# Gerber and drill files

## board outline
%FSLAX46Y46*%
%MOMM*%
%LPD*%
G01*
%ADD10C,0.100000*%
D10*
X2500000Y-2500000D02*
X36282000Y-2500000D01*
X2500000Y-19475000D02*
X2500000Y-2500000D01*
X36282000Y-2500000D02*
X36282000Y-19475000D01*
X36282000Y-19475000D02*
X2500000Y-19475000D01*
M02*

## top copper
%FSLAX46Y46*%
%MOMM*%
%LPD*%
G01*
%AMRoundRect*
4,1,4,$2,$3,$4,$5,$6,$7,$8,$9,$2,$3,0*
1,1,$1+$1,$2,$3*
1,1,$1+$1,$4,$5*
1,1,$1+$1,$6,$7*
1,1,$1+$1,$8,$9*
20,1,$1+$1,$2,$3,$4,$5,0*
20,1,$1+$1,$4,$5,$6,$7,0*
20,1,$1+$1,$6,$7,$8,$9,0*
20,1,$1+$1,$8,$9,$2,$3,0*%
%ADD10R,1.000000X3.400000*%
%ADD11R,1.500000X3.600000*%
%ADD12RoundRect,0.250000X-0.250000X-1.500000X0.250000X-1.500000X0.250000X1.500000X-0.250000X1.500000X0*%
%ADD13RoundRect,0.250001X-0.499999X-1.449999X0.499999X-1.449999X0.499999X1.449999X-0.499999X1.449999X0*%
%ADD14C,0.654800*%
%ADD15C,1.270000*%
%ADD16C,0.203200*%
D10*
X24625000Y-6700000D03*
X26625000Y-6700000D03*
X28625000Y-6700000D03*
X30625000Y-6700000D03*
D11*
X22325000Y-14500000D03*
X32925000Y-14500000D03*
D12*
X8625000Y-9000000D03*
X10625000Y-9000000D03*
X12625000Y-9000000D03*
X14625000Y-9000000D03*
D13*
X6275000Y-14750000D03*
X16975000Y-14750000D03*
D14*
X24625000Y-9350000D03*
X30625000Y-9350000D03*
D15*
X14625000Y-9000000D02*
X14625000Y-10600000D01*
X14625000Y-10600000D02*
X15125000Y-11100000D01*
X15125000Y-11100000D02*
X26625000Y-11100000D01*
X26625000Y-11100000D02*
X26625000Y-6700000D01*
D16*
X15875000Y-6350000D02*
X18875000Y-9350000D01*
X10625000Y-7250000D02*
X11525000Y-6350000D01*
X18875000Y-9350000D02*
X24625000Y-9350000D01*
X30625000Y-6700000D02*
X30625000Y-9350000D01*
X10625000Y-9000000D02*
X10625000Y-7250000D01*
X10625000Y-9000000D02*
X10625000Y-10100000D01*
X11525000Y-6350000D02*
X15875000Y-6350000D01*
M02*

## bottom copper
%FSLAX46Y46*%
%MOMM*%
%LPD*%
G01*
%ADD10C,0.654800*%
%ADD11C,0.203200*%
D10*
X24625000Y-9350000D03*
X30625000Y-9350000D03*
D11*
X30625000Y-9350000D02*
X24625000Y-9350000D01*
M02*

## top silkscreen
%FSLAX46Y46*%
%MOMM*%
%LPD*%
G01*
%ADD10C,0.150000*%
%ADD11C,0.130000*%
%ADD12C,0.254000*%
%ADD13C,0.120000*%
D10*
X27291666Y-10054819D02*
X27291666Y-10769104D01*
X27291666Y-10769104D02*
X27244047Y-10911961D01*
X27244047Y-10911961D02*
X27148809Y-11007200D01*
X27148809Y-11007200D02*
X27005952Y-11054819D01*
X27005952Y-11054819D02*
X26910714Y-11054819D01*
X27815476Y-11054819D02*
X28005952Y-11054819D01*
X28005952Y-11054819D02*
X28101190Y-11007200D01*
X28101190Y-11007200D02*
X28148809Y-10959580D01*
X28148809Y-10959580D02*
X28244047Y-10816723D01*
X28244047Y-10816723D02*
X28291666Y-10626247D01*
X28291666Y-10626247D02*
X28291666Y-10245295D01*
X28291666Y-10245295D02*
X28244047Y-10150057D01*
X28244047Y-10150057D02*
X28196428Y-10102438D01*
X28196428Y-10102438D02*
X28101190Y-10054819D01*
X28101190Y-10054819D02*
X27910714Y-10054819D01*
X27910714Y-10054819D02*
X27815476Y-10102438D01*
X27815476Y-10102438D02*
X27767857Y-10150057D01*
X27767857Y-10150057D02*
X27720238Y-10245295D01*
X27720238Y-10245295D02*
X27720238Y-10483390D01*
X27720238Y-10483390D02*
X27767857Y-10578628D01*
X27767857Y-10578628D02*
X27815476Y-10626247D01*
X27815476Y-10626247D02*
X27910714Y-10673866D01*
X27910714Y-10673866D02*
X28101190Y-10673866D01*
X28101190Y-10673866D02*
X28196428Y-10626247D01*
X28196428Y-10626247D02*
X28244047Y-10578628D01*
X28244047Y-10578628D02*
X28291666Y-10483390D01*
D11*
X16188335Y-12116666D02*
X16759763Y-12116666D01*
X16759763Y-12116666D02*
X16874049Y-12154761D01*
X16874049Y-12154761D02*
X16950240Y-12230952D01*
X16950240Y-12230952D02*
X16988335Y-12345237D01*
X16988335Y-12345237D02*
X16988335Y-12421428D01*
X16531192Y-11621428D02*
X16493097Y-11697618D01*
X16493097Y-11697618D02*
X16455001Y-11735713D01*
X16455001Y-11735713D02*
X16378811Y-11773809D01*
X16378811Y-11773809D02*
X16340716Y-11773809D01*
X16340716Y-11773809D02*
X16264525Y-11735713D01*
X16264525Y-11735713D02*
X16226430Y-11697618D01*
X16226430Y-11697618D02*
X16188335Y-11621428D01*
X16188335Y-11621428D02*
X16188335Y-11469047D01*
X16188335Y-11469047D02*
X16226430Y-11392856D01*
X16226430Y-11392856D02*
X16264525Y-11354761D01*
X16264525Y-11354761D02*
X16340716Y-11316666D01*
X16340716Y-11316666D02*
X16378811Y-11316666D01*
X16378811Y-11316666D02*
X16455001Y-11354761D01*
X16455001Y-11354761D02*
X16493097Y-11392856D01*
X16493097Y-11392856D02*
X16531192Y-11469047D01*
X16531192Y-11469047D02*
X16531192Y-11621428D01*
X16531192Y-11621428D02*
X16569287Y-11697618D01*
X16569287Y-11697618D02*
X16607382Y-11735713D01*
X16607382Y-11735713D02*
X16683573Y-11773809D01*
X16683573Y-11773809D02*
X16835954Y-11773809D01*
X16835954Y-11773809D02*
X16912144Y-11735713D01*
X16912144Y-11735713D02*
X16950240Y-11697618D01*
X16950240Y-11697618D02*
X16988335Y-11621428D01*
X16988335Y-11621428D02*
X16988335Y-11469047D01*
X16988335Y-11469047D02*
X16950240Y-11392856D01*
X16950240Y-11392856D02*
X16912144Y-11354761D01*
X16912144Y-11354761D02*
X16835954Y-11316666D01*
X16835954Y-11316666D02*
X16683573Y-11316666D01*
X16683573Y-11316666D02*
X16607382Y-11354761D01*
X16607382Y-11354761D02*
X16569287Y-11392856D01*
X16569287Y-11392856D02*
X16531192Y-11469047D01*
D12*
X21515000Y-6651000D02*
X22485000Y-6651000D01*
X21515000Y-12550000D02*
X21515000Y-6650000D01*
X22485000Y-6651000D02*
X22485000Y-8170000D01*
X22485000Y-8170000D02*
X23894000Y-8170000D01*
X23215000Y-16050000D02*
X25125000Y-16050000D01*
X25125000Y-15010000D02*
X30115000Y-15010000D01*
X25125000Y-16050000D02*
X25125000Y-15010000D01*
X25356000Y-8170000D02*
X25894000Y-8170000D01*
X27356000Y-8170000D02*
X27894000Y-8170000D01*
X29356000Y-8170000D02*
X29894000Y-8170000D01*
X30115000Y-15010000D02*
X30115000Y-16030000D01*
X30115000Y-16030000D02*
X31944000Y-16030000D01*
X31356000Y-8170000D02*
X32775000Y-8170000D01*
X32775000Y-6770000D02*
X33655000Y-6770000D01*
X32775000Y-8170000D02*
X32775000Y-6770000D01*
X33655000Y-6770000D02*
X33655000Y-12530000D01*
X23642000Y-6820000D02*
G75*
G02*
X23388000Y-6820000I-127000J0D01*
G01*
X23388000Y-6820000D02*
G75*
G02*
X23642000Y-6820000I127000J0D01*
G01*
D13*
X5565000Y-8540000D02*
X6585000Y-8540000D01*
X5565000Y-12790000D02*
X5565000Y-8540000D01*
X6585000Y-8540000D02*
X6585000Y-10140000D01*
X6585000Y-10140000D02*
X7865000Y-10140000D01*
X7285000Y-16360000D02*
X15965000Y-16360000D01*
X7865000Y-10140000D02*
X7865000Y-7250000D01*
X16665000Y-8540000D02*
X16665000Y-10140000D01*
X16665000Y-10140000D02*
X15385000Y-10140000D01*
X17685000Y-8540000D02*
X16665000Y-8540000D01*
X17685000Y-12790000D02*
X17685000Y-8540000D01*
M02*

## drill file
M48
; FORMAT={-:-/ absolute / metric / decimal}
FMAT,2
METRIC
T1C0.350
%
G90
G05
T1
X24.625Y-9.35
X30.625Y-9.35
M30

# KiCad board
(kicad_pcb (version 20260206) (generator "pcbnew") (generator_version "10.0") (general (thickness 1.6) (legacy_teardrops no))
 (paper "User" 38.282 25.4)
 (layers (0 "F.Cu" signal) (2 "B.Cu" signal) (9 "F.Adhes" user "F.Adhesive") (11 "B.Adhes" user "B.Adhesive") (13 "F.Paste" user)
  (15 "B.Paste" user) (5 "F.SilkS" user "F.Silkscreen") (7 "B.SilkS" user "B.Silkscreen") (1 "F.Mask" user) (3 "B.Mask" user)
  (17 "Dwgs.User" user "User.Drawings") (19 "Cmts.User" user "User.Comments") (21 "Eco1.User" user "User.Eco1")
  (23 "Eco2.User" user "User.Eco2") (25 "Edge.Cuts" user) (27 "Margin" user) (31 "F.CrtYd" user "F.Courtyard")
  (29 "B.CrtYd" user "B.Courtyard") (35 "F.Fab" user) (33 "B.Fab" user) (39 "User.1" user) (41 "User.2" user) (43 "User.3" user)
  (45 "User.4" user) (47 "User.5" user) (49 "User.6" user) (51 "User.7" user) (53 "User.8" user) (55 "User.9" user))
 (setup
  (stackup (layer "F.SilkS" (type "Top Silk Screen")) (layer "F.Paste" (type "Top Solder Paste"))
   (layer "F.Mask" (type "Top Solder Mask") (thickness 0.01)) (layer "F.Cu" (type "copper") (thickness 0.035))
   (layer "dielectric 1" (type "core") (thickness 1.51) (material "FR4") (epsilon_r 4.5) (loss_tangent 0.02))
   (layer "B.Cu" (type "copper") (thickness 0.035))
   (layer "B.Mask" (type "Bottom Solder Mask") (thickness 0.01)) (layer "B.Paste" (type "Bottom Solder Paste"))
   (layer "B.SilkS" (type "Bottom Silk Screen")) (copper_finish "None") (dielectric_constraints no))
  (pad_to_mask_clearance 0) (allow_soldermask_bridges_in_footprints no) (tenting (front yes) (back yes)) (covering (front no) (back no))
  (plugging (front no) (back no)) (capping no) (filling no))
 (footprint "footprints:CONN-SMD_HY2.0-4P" (layer "F.Cu") (at 27.625 10.6)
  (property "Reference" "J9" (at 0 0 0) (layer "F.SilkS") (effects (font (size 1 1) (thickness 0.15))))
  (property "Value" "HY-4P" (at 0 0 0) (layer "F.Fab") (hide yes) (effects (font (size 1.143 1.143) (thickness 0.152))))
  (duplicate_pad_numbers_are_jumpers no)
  (fp_line (start -6.11 -3.949) (end -5.14 -3.949) (stroke (width 0.254) (type solid)) (layer "F.SilkS"))
  (fp_line (start -6.11 1.95) (end -6.11 -3.95) (stroke (width 0.254) (type solid)) (layer "F.SilkS"))
  (fp_line (start -5.14 -3.949) (end -5.14 -2.43) (stroke (width 0.254) (type solid)) (layer "F.SilkS"))
  (fp_line (start -5.14 -2.43) (end -3.731 -2.43) (stroke (width 0.254) (type solid)) (layer "F.SilkS"))
  (fp_line (start -4.41 5.45) (end -2.5 5.45) (stroke (width 0.254) (type solid)) (layer "F.SilkS"))
  (fp_line (start -2.5 4.41) (end 2.49 4.41) (stroke (width 0.254) (type solid)) (layer "F.SilkS"))
  (fp_line (start -2.5 5.45) (end -2.5 4.41) (stroke (width 0.254) (type solid)) (layer "F.SilkS"))
  (fp_line (start -2.269 -2.43) (end -1.731 -2.43) (stroke (width 0.254) (type solid)) (layer "F.SilkS"))
  (fp_line (start -0.269 -2.43) (end 0.269 -2.43) (stroke (width 0.254) (type solid)) (layer "F.SilkS"))
  (fp_line (start 1.731 -2.43) (end 2.269 -2.43) (stroke (width 0.254) (type solid)) (layer "F.SilkS"))
  (fp_line (start 2.49 4.41) (end 2.49 5.43) (stroke (width 0.254) (type solid)) (layer "F.SilkS"))
  (fp_line (start 2.49 5.43) (end 4.319 5.43) (stroke (width 0.254) (type solid)) (layer "F.SilkS"))
  (fp_line (start 3.731 -2.43) (end 5.15 -2.43) (stroke (width 0.254) (type solid)) (layer "F.SilkS"))
  (fp_line (start 5.15 -3.83) (end 6.03 -3.83) (stroke (width 0.254) (type solid)) (layer "F.SilkS"))
  (fp_line (start 5.15 -2.43) (end 5.15 -3.83) (stroke (width 0.254) (type solid)) (layer "F.SilkS"))
  (fp_line (start 6.03 -3.83) (end 6.03 1.93) (stroke (width 0.254) (type solid)) (layer "F.SilkS"))
  (fp_circle (center -4.11 -3.78) (end -3.983 -3.78) (stroke (width 0.254) (type solid)) (fill no) (layer "F.SilkS"))
  (pad "1" smd rect (at -3 -3.9 180) (size 1 3.4) (layers "F.Cu" "F.Mask" "F.Paste") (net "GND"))
  (pad "2" smd rect (at -1 -3.9 180) (size 1 3.4) (layers "F.Cu" "F.Mask" "F.Paste") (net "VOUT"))
  (pad "3" smd rect (at 1 -3.9 180) (size 1 3.4) (layers "F.Cu" "F.Mask" "F.Paste") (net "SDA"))
  (pad "4" smd rect (at 3 -3.9 180) (size 1 3.4) (layers "F.Cu" "F.Mask" "F.Paste") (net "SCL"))
  (pad "MP" smd rect (at -5.3 3.9 180) (size 1.5 3.6) (layers "F.Cu" "F.Mask" "F.Paste") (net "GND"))
  (pad "MP" smd rect (at 5.3 3.9 180) (size 1.5 3.6) (layers "F.Cu" "F.Mask" "F.Paste") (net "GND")))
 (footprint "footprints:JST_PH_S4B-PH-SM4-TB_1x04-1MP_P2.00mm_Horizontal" (layer "F.Cu") (at 11.625 11.85)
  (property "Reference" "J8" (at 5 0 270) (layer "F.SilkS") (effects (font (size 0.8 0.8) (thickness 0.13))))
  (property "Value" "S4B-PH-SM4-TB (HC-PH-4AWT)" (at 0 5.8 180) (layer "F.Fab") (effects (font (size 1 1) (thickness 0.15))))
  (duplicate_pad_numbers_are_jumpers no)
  (fp_line (start -6.06 -3.31) (end -5.04 -3.31) (stroke (width 0.12) (type solid)) (layer "F.SilkS"))
  (fp_line (start -6.06 0.94) (end -6.06 -3.31) (stroke (width 0.12) (type solid)) (layer "F.SilkS"))
  (fp_line (start -5.04 -3.31) (end -5.04 -1.71) (stroke (width 0.12) (type solid)) (layer "F.SilkS"))
  (fp_line (start -5.04 -1.71) (end -3.76 -1.71) (stroke (width 0.12) (type solid)) (layer "F.SilkS"))
  (fp_line (start -4.34 4.51) (end 4.34 4.51) (stroke (width 0.12) (type solid)) (layer "F.SilkS"))
  (fp_line (start -3.76 -1.71) (end -3.76 -4.6) (stroke (width 0.12) (type solid)) (layer "F.SilkS"))
  (fp_line (start 5.04 -3.31) (end 5.04 -1.71) (stroke (width 0.12) (type solid)) (layer "F.SilkS"))
  (fp_line (start 5.04 -1.71) (end 3.76 -1.71) (stroke (width 0.12) (type solid)) (layer "F.SilkS"))
  (fp_line (start 6.06 -3.31) (end 5.04 -3.31) (stroke (width 0.12) (type solid)) (layer "F.SilkS"))
  (fp_line (start 6.06 0.94) (end 6.06 -3.31) (stroke (width 0.12) (type solid)) (layer "F.SilkS"))
  (pad "1" smd roundrect (at -3 -2.85) (size 1 3.5) (layers "F.Cu" "F.Mask" "F.Paste") (roundrect_rratio 0.25) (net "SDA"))
  (pad "2" smd roundrect (at -1 -2.85) (size 1 3.5) (layers "F.Cu" "F.Mask" "F.Paste") (roundrect_rratio 0.25) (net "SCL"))
  (pad "3" smd roundrect (at 1 -2.85) (size 1 3.5) (layers "F.Cu" "F.Mask" "F.Paste") (roundrect_rratio 0.25) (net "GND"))
  (pad "4" smd roundrect (at 3 -2.85) (size 1 3.5) (layers "F.Cu" "F.Mask" "F.Paste") (roundrect_rratio 0.25) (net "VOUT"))
  (pad "MP" smd roundrect (at -5.35 2.9) (size 1.5 3.4) (layers "F.Cu" "F.Mask" "F.Paste") (roundrect_rratio 0.166667) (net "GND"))
  (pad "MP" smd roundrect (at 5.35 2.9) (size 1.5 3.4) (layers "F.Cu" "F.Mask" "F.Paste") (roundrect_rratio 0.166667) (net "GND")))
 (gr_line (start 2.5 2.5) (end 36.282 2.5) (stroke (width 0.1) (type default)) (layer "Edge.Cuts"))
 (gr_line (start 2.5 19.475) (end 2.5 2.5) (stroke (width 0.1) (type default)) (layer "Edge.Cuts"))
 (gr_line (start 36.282 2.5) (end 36.282 19.475) (stroke (width 0.1) (type default)) (layer "Edge.Cuts"))
 (gr_line (start 36.282 19.475) (end 2.5 19.475) (stroke (width 0.1) (type default)) (layer "Edge.Cuts"))
 (segment (start 14.625 9) (end 14.625 10.6) (width 1.27) (layer "F.Cu") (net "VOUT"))
 (segment (start 14.625 10.6) (end 15.125 11.1) (width 1.27) (layer "F.Cu") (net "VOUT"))
 (segment (start 15.125 11.1) (end 26.625 11.1) (width 1.27) (layer "F.Cu") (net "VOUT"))
 (segment (start 26.625 11.1) (end 26.625 6.7) (width 1.27) (layer "F.Cu") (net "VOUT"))
 (segment (start 15.875 6.35) (end 18.875 9.35) (width 0.2032) (layer "F.Cu") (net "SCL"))
 (segment (start 10.625 7.25) (end 11.525 6.35) (width 0.2032) (layer "F.Cu") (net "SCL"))
 (segment (start 18.875 9.35) (end 24.625 9.35) (width 0.2032) (layer "F.Cu") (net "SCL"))
 (segment (start 30.625 6.7) (end 30.625 9.35) (width 0.2032) (layer "F.Cu") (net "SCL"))
 (segment (start 10.625 9) (end 10.625 7.25) (width 0.2032) (layer "F.Cu") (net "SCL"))
 (segment (start 10.625 9) (end 10.625 10.1) (width 0.2032) (layer "F.Cu") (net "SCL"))
 (segment (start 11.525 6.35) (end 15.875 6.35) (width 0.2032) (layer "F.Cu") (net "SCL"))
 (via (at 24.625 9.35) (size 0.6548) (drill 0.35) (layers "F.Cu" "B.Cu") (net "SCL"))
 (via (at 30.625 9.35) (size 0.6548) (drill 0.35) (layers "F.Cu" "B.Cu") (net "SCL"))
 (segment (start 30.625 9.35) (end 24.625 9.35) (width 0.2032) (layer "B.Cu") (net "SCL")))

